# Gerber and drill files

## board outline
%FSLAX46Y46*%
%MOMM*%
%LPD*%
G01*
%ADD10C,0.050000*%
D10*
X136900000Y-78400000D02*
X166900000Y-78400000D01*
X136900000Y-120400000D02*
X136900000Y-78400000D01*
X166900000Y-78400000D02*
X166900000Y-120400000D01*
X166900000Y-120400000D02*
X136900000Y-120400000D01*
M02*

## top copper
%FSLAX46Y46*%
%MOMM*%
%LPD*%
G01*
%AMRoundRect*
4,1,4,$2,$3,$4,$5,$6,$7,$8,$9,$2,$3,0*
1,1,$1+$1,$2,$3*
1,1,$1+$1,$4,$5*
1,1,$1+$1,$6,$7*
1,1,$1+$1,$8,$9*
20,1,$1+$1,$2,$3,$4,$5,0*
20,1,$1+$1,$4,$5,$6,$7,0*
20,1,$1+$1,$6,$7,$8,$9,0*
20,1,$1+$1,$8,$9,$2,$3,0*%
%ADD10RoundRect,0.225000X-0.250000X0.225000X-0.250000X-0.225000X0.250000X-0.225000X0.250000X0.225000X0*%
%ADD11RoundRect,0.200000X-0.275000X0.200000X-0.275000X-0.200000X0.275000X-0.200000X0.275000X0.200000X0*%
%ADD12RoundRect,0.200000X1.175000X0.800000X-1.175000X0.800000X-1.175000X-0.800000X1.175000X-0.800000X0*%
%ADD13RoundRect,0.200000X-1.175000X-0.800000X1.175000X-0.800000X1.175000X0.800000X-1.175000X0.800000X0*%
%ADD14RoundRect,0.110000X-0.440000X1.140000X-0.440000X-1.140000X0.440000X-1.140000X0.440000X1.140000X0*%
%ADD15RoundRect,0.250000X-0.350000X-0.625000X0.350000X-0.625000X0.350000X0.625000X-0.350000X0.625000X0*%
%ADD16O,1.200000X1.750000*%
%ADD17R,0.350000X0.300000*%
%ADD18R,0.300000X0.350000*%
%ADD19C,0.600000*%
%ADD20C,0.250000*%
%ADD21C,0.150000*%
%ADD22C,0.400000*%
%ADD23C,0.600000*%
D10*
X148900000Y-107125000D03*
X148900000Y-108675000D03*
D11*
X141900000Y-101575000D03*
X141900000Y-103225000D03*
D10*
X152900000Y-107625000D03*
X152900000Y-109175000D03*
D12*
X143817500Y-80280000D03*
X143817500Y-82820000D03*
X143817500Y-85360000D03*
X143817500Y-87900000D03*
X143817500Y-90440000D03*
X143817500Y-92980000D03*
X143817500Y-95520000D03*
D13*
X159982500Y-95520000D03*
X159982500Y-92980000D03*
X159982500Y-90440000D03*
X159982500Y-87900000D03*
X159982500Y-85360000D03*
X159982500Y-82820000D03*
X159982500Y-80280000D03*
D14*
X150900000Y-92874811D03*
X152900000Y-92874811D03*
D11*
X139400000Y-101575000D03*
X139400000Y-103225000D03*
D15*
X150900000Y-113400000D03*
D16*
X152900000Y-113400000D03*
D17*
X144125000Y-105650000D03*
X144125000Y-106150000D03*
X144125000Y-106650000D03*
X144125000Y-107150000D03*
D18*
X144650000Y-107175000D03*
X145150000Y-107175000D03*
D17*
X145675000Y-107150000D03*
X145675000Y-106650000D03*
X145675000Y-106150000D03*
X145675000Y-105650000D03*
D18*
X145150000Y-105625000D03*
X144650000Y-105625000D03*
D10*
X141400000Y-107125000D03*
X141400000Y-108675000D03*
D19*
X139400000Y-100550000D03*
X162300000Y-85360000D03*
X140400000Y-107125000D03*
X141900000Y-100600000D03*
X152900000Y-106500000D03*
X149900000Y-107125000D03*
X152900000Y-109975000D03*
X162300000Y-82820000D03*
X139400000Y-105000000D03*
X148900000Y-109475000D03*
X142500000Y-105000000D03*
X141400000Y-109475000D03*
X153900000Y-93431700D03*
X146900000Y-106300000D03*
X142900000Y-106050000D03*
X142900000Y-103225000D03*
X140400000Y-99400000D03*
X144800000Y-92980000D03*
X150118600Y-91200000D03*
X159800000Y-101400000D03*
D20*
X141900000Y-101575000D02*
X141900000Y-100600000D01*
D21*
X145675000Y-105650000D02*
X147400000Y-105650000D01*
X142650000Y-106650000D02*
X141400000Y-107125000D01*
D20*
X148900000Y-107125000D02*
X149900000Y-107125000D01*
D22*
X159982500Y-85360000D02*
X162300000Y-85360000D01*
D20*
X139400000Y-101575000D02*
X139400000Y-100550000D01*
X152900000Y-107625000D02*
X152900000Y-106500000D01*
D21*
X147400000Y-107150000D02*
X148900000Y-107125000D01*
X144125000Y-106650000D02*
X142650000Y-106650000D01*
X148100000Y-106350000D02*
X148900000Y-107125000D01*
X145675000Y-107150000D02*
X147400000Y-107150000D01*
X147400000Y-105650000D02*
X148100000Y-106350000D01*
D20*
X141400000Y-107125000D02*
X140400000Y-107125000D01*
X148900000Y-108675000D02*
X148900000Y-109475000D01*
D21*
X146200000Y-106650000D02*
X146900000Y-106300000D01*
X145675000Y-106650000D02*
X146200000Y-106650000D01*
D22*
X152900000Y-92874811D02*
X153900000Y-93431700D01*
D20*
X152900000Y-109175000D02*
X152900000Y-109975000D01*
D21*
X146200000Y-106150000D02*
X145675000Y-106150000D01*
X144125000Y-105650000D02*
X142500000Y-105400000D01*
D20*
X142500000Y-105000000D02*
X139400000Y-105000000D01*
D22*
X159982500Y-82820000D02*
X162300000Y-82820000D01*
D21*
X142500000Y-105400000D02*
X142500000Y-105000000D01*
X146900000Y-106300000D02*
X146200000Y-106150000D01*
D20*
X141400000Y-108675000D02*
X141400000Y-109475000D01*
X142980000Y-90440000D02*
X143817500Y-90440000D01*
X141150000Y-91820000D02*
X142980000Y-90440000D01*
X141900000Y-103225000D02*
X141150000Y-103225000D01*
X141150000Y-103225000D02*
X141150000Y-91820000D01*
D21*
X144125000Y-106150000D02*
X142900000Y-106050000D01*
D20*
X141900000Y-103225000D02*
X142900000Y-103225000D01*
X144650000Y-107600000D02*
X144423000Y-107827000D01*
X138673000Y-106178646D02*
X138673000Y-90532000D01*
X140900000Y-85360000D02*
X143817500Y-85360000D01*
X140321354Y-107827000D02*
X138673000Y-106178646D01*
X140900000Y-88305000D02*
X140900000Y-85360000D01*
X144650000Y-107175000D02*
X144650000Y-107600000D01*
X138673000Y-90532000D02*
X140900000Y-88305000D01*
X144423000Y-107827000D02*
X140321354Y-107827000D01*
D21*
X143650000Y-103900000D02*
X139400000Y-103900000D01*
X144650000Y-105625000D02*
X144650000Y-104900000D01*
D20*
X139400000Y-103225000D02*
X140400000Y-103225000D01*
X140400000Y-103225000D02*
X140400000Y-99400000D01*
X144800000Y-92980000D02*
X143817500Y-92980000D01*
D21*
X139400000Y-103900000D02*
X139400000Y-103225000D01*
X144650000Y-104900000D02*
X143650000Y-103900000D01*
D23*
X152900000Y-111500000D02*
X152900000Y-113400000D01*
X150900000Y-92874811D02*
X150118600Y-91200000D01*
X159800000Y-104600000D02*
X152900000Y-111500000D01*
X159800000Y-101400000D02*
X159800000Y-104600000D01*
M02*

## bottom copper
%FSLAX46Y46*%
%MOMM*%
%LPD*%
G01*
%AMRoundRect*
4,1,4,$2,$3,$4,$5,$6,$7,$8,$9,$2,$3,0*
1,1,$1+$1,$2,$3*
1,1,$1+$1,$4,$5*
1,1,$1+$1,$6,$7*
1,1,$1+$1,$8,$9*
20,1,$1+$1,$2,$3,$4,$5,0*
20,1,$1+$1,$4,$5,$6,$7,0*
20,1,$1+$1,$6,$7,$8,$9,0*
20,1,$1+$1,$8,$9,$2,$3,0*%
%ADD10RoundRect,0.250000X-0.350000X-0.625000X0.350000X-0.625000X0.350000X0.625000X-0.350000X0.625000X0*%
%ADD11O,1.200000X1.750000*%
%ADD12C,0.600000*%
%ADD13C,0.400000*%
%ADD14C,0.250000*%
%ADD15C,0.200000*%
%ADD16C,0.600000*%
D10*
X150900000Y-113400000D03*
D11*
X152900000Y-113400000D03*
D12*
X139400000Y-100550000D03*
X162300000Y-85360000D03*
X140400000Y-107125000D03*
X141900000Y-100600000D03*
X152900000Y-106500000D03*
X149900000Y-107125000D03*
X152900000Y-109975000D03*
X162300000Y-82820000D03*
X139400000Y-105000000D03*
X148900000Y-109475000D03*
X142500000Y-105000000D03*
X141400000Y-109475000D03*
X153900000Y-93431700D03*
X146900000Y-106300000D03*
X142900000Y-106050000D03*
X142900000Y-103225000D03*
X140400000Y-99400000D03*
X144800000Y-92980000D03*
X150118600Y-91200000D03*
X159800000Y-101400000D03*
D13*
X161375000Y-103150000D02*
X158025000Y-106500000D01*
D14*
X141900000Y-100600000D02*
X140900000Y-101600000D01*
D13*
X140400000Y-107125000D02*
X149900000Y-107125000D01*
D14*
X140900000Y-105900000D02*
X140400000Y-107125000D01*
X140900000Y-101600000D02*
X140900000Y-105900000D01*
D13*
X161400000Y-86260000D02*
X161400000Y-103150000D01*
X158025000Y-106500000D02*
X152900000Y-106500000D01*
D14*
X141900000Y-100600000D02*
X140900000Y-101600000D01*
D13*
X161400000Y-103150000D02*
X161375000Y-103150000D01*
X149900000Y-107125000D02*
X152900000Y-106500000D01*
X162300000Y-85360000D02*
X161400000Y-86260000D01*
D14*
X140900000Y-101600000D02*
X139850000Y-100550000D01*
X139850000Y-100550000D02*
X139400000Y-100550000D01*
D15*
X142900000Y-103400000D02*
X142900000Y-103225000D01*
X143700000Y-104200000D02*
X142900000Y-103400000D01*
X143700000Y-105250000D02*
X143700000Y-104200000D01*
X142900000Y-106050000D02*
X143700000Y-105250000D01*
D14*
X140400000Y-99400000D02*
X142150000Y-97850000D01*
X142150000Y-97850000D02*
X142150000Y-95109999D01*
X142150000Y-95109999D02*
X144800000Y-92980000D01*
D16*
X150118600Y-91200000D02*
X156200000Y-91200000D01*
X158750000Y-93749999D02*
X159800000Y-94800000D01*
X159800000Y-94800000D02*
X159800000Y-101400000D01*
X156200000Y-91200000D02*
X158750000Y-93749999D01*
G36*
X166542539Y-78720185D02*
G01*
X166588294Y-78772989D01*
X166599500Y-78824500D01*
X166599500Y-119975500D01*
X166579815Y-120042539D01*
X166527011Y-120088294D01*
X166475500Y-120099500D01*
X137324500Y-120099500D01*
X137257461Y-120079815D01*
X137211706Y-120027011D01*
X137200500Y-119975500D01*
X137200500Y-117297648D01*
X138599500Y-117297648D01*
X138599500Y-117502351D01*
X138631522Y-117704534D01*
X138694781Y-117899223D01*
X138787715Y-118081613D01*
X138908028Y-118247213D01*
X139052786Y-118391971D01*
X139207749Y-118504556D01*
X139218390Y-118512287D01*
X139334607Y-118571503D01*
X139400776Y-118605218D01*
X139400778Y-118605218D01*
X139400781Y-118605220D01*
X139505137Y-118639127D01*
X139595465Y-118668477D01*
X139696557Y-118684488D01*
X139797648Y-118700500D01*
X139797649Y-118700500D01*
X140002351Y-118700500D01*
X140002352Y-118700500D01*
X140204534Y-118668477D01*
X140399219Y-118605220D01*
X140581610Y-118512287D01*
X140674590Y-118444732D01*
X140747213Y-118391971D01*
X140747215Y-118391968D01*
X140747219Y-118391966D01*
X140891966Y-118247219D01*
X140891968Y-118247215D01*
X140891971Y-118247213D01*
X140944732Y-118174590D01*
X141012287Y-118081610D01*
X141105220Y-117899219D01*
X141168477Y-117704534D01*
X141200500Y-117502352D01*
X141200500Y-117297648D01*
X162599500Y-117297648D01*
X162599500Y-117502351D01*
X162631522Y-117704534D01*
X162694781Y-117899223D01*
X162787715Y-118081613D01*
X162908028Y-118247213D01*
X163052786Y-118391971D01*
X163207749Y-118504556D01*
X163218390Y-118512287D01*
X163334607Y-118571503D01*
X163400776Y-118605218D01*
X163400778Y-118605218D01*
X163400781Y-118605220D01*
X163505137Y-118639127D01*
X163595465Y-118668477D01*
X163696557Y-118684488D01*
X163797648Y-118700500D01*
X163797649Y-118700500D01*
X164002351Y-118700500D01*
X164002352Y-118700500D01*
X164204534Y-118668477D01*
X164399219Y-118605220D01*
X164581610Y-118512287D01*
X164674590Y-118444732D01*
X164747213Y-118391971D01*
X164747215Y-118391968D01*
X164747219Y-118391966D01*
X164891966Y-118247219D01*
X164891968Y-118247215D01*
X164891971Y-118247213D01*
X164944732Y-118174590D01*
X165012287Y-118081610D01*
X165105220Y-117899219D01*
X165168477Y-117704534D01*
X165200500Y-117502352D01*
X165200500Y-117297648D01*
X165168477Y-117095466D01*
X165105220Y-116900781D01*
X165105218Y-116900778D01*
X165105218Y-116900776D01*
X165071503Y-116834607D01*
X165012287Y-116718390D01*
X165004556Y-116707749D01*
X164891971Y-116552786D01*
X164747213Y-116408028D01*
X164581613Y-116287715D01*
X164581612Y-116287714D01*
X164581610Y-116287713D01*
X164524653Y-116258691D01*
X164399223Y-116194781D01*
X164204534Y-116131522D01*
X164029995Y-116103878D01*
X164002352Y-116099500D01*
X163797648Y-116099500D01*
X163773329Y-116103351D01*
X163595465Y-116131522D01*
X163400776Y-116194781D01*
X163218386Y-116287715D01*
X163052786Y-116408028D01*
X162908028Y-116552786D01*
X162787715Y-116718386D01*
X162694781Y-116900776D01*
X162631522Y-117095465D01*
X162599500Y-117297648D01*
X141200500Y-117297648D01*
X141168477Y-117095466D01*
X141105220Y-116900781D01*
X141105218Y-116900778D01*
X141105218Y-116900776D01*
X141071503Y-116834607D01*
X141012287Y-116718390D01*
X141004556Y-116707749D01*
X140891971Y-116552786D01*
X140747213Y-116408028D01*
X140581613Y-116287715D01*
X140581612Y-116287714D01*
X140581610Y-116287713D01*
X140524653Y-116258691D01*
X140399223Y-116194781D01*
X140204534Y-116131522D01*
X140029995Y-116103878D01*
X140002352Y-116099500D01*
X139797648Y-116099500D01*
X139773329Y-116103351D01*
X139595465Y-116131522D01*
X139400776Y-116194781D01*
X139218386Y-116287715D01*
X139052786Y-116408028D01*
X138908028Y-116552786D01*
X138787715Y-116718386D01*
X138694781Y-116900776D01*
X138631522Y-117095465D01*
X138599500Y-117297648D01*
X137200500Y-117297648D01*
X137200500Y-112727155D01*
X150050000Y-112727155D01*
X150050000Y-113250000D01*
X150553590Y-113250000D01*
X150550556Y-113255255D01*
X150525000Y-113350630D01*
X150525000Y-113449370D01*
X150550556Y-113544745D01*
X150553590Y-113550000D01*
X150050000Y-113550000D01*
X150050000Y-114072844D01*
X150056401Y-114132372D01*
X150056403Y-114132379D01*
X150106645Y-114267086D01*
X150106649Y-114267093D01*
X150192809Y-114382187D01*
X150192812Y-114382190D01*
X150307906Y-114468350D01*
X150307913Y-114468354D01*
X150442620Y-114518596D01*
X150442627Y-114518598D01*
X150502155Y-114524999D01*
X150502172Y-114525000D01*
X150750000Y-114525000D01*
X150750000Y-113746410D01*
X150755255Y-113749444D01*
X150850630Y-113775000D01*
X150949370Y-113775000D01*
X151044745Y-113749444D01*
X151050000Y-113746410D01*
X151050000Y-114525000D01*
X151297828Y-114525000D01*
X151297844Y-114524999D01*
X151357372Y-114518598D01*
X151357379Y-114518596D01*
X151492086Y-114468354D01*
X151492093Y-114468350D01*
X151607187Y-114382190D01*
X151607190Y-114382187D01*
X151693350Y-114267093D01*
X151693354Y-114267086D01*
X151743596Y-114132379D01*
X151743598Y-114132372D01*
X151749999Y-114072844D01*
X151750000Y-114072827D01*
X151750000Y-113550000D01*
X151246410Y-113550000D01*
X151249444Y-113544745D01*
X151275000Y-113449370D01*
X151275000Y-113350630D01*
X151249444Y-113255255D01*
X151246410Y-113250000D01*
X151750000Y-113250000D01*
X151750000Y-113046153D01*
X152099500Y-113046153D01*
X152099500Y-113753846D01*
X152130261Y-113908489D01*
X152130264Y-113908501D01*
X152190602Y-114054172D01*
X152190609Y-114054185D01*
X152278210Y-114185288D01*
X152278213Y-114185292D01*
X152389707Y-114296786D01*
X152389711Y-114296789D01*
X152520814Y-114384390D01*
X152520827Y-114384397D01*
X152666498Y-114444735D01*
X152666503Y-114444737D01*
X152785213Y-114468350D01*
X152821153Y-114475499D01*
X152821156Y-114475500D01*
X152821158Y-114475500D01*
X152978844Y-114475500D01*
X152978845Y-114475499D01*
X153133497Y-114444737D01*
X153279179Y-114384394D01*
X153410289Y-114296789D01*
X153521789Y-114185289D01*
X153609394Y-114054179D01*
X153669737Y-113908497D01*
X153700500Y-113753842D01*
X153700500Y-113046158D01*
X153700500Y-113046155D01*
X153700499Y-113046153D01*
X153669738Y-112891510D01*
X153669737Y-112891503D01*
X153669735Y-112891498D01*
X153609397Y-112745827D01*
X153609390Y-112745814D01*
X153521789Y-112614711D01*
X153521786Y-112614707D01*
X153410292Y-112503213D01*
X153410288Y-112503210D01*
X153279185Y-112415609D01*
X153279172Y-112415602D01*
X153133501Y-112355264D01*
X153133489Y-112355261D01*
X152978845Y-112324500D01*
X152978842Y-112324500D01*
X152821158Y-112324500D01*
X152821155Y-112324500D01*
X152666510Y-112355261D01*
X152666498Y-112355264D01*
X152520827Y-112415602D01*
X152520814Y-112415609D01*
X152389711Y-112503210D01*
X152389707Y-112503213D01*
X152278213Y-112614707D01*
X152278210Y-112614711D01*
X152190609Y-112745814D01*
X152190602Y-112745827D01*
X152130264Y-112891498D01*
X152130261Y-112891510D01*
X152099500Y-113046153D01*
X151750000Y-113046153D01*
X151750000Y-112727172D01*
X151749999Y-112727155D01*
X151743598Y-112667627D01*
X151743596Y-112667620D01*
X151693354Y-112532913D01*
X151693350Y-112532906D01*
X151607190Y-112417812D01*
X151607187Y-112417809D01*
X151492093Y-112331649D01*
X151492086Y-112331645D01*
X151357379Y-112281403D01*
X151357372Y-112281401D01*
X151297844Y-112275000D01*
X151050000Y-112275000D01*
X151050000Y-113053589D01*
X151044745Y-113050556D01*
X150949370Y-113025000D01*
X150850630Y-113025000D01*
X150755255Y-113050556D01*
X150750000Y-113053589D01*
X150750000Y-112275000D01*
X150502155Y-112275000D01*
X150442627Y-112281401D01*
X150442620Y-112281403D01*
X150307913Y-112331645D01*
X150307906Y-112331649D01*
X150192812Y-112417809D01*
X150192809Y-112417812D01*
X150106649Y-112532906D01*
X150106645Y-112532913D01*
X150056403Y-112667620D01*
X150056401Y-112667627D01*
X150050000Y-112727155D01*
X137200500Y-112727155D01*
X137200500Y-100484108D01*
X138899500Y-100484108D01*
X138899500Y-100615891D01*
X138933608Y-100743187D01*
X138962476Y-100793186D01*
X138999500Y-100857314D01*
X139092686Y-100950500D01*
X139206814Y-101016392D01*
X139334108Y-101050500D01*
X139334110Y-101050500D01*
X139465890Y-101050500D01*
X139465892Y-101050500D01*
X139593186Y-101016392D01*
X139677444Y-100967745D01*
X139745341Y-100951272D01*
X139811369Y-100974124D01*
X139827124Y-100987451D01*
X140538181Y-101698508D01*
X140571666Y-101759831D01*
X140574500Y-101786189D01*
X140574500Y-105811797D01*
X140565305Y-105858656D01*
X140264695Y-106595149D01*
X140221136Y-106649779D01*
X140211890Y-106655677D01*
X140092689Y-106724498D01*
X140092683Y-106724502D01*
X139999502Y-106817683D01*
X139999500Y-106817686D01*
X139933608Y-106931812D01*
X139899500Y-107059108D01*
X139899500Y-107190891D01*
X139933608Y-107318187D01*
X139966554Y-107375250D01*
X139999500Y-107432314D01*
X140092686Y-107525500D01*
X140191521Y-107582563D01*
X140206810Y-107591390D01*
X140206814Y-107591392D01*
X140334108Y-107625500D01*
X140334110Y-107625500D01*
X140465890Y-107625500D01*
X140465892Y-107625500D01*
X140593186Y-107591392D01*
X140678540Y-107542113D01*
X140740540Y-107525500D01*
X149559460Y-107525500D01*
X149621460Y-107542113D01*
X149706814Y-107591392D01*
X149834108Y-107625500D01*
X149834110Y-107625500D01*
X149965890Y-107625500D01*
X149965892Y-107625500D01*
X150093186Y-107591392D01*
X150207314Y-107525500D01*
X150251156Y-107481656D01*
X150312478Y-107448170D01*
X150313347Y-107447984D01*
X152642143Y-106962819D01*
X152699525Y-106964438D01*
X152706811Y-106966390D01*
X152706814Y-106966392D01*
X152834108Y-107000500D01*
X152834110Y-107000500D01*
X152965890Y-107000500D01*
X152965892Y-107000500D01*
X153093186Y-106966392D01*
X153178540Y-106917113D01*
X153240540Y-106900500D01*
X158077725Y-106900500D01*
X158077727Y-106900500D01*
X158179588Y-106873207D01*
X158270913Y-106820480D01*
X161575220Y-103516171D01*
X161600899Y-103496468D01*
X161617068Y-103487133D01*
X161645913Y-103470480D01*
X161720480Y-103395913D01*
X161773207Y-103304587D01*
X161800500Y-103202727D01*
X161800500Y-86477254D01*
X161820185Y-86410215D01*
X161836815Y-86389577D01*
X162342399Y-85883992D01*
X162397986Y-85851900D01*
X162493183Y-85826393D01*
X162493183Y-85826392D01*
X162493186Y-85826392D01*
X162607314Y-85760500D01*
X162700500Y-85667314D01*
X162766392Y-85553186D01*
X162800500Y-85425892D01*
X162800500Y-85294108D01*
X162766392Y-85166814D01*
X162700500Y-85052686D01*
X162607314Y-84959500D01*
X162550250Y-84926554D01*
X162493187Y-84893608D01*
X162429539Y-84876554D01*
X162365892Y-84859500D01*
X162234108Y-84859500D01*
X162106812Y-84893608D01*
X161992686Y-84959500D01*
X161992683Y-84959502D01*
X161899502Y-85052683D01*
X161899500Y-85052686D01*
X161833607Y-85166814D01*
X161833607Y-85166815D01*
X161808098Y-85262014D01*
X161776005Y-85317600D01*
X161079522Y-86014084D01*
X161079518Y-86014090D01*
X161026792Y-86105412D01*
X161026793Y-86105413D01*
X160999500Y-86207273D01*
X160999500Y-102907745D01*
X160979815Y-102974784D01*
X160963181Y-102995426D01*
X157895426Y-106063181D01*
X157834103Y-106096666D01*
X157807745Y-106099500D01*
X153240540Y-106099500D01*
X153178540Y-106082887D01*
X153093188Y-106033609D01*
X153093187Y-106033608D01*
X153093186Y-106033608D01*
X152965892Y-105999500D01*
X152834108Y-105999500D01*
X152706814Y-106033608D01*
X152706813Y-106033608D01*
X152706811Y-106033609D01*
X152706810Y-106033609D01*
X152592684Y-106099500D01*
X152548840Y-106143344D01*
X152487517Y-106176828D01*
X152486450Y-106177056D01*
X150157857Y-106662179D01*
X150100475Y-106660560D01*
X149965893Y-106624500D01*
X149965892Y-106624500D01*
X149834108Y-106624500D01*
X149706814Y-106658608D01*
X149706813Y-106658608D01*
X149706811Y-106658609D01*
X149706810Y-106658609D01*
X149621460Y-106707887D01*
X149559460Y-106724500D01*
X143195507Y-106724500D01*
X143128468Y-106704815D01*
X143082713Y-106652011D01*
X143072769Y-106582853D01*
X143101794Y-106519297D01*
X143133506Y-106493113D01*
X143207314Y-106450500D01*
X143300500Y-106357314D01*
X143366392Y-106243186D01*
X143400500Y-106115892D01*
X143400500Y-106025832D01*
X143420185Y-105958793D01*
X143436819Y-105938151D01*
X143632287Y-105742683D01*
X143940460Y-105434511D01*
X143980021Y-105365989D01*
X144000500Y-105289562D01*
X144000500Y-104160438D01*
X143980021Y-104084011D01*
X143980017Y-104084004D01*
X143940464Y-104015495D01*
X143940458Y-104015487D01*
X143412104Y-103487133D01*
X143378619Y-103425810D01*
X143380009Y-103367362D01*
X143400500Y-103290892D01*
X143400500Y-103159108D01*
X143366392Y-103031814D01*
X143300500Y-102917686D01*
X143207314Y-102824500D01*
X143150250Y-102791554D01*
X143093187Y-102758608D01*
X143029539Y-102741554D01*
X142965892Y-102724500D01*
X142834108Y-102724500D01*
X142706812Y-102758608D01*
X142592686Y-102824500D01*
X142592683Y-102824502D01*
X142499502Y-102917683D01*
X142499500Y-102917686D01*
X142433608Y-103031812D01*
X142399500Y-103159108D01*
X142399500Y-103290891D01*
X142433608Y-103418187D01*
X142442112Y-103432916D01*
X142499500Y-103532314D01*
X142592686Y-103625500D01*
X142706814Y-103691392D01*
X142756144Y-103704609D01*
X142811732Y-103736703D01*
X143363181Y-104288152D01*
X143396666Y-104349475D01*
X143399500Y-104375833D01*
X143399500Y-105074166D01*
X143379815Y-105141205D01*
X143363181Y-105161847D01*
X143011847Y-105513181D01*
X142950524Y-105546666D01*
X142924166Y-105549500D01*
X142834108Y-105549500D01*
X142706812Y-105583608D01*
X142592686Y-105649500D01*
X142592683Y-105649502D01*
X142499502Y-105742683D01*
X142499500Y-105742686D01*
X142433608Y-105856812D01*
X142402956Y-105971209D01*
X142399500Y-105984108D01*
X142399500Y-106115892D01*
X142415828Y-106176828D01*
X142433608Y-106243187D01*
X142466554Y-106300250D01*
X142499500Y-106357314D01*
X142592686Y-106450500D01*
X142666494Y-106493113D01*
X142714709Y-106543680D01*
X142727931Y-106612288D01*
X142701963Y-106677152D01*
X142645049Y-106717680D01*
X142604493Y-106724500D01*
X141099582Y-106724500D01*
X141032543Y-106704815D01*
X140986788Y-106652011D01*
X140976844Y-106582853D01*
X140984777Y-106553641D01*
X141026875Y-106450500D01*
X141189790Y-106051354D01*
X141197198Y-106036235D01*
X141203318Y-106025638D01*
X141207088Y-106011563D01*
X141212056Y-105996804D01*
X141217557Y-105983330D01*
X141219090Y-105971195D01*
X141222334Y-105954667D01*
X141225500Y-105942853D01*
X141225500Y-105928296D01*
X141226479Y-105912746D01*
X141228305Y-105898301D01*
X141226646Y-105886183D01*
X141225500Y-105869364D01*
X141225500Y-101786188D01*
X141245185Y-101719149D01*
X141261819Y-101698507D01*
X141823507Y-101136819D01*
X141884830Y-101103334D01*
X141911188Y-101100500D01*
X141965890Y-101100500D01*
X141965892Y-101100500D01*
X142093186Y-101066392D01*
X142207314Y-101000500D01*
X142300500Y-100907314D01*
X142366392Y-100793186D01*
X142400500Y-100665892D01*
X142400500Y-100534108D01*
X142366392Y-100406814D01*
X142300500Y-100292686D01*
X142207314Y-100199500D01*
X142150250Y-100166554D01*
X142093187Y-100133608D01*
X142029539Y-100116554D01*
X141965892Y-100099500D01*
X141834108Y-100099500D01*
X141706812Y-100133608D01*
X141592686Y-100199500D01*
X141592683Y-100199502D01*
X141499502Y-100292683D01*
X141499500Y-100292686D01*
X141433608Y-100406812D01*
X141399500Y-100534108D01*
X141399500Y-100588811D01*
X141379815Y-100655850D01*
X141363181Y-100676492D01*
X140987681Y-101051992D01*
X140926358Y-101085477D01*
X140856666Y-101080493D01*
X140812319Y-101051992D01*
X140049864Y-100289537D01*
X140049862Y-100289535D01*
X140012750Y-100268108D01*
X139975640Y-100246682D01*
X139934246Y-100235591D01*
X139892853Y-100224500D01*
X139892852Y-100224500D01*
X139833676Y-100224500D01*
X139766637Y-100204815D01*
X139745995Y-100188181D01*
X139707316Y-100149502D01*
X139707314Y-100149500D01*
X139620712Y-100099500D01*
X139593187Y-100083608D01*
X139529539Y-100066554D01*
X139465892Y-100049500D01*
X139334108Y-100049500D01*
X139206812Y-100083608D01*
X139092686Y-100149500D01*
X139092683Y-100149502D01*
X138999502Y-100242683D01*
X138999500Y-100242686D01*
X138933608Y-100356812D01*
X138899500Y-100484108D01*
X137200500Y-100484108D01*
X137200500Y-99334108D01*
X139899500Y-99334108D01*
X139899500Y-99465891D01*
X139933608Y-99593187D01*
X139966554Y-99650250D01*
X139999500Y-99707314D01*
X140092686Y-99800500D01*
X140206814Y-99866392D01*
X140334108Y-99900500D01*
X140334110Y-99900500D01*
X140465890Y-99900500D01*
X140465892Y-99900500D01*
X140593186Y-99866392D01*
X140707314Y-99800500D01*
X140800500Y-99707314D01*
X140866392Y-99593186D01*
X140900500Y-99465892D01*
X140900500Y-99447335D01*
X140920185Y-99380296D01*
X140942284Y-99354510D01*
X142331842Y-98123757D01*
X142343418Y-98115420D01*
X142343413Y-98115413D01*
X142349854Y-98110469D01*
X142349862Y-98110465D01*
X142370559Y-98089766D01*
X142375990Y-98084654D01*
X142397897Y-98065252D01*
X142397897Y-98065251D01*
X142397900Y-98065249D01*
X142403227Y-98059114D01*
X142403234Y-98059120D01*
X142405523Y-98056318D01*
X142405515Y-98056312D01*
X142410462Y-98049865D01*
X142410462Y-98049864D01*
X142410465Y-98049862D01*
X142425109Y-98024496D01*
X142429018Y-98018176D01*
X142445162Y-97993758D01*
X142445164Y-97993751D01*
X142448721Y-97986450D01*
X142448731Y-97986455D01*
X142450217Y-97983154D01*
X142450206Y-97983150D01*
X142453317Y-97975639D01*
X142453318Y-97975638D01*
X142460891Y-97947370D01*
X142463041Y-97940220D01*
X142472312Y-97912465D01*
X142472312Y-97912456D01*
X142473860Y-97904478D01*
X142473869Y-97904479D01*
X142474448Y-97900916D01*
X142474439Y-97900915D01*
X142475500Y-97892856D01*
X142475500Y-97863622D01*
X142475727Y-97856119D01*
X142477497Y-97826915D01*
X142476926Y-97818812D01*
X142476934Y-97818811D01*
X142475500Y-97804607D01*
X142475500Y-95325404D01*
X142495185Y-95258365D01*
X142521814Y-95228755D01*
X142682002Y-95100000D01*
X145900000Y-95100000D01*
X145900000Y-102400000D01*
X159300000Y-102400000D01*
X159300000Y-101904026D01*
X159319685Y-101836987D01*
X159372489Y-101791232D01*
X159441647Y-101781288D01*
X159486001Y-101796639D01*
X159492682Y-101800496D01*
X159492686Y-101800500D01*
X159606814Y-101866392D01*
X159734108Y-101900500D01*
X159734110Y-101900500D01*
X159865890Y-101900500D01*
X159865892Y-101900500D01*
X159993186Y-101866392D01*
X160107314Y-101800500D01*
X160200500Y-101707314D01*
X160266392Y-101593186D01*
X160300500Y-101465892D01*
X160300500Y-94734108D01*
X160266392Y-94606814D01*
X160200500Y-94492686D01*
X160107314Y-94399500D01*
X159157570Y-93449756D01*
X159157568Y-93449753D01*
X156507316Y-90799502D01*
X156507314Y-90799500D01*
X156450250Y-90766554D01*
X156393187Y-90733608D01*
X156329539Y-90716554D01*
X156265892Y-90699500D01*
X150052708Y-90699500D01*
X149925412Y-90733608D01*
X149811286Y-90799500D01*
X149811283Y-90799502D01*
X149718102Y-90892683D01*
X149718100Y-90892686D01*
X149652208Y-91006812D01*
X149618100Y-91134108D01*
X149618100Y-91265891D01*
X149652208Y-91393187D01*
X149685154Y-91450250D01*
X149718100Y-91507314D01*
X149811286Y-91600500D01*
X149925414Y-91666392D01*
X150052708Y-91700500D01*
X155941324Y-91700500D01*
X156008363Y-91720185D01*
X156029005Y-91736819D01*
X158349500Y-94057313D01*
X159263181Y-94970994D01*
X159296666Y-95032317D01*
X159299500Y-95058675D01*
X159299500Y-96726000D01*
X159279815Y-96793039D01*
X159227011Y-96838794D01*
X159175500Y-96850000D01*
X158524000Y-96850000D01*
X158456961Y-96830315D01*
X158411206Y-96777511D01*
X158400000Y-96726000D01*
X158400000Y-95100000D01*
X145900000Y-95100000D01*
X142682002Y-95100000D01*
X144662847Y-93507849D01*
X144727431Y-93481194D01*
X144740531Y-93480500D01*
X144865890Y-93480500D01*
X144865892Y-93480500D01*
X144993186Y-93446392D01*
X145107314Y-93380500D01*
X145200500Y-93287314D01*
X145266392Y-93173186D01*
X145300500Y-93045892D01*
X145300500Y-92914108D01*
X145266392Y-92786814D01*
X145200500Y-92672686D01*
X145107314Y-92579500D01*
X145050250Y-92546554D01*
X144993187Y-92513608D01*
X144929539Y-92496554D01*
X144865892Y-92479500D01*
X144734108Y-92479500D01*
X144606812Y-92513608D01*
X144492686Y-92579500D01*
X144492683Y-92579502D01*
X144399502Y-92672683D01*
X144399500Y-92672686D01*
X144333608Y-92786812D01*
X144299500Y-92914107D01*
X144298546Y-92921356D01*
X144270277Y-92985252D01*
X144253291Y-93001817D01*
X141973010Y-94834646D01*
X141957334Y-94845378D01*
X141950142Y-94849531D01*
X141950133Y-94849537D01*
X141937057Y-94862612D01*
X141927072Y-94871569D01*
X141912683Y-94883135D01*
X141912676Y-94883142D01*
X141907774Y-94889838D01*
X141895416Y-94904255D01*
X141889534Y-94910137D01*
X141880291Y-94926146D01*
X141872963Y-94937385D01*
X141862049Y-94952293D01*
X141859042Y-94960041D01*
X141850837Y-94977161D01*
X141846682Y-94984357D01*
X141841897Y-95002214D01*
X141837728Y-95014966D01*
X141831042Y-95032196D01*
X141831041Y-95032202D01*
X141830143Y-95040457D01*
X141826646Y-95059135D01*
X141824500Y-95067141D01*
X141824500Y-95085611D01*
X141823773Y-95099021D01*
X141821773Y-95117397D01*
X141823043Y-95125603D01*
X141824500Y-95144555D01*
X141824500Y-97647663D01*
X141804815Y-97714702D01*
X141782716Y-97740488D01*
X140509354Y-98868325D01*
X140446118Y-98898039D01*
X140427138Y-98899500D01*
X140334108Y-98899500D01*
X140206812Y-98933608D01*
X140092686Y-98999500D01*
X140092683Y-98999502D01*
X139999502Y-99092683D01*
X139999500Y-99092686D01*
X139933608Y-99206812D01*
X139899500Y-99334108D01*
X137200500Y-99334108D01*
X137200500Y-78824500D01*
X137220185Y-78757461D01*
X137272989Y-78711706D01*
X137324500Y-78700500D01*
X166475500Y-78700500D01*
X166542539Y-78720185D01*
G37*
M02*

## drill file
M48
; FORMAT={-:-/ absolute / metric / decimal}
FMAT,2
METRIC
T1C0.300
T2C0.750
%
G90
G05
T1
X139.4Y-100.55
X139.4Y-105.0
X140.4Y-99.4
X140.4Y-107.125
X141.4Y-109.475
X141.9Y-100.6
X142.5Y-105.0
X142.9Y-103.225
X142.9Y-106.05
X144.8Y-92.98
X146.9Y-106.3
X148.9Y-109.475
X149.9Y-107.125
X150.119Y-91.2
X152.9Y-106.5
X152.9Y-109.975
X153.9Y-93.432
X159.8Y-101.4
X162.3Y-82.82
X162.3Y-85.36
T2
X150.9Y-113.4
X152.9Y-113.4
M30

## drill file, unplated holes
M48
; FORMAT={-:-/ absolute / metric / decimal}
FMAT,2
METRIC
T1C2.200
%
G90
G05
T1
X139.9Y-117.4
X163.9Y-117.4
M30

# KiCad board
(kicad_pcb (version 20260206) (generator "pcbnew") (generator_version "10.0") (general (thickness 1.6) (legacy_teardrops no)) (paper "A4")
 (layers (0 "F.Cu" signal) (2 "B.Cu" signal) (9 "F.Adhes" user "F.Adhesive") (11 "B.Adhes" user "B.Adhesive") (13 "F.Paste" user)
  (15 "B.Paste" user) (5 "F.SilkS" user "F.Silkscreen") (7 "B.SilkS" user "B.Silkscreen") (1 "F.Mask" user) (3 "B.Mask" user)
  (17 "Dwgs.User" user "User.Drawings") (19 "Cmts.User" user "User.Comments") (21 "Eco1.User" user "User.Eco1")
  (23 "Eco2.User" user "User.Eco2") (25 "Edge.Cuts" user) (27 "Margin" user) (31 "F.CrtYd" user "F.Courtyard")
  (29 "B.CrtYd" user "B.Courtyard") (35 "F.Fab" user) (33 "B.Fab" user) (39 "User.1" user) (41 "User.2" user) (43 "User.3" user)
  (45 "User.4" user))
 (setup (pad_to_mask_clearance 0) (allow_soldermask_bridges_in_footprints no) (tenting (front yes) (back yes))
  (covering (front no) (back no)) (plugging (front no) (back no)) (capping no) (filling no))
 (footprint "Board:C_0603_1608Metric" (layer "F.Cu") (at 148.9 107.9 -90)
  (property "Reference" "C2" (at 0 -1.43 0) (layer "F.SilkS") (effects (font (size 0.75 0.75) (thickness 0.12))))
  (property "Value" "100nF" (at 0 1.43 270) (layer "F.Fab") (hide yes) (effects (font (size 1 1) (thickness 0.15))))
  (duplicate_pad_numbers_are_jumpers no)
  (pad "1" smd roundrect (at -0.775 0 270) (size 0.9 0.95) (layers "F.Cu" "F.Mask" "F.Paste") (roundrect_rratio 0.25) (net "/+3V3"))
  (pad "2" smd roundrect (at 0.775 0 270) (size 0.9 0.95) (layers "F.Cu" "F.Mask" "F.Paste") (roundrect_rratio 0.25) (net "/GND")))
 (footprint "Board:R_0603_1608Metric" (layer "F.Cu") (at 141.9 102.4 -90)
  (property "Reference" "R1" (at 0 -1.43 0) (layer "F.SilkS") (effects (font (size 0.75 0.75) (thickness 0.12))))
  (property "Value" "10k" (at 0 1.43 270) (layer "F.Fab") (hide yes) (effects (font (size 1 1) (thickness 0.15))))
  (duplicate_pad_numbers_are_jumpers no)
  (pad "1" smd roundrect (at -0.825 0 270) (size 0.8 0.95) (layers "F.Cu" "F.Mask" "F.Paste") (roundrect_rratio 0.25) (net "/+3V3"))
  (pad "2" smd roundrect (at 0.825 0 270) (size 0.8 0.95) (layers "F.Cu" "F.Mask" "F.Paste") (roundrect_rratio 0.25) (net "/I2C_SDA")))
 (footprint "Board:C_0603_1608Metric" (layer "F.Cu") (at 152.9 108.4 -90)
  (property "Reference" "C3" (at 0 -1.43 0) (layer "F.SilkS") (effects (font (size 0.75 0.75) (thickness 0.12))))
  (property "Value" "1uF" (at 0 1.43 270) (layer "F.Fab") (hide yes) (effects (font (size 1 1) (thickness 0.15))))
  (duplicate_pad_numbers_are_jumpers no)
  (pad "1" smd roundrect (at -0.775 0 270) (size 0.9 0.95) (layers "F.Cu" "F.Mask" "F.Paste") (roundrect_rratio 0.25) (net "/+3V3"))
  (pad "2" smd roundrect (at 0.775 0 270) (size 0.9 0.95) (layers "F.Cu" "F.Mask" "F.Paste") (roundrect_rratio 0.25) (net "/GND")))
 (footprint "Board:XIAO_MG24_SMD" (layer "F.Cu") (at 151.9 87.9 90)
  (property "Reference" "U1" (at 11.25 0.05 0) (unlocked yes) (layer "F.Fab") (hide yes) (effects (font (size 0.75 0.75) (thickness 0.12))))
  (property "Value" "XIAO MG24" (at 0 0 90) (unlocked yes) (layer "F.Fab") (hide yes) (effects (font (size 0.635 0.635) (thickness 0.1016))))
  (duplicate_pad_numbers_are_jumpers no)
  (pad "1" smd roundrect (at 7.62 -8.0825 180) (size 2.75 2) (layers "F.Cu" "F.Mask" "F.Paste") (roundrect_rratio 0.1)
   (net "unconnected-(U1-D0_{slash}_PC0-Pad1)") (thermal_bridge_angle 45))
  (pad "2" smd roundrect (at 5.08 -8.0825 180) (size 2.75 2) (layers "F.Cu" "F.Mask" "F.Paste") (roundrect_rratio 0.1)
   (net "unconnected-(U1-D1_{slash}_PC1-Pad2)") (thermal_bridge_angle 45))
  (pad "3" smd roundrect (at 2.54 -8.0825 180) (size 2.75 2) (layers "F.Cu" "F.Mask" "F.Paste") (roundrect_rratio 0.1) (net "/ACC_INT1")
   (thermal_bridge_angle 45))
  (pad "4" smd roundrect (at 0 -8.0825 180) (size 2.75 2) (layers "F.Cu" "F.Mask" "F.Paste") (roundrect_rratio 0.1)
   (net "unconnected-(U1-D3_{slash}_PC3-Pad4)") (thermal_bridge_angle 45))
  (pad "5" smd roundrect (at -2.54 -8.0825 180) (size 2.75 2) (layers "F.Cu" "F.Mask" "F.Paste") (roundrect_rratio 0.1) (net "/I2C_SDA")
   (thermal_bridge_angle 45))
  (pad "6" smd roundrect (at -5.08 -8.0825 180) (size 2.75 2) (layers "F.Cu" "F.Mask" "F.Paste") (roundrect_rratio 0.1) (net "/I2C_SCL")
   (thermal_bridge_angle 45))
  (pad "7" smd roundrect (at -7.62 -8.0825 180) (size 2.75 2) (layers "F.Cu" "F.Mask" "F.Paste") (roundrect_rratio 0.1)
   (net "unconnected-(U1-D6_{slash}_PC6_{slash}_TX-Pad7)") (thermal_bridge_angle 45))
  (pad "8" smd roundrect (at -7.62 8.0825) (size 2.75 2) (layers "F.Cu" "F.Mask" "F.Paste") (roundrect_rratio 0.1)
   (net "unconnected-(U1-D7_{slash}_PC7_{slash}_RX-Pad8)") (thermal_bridge_angle 45))
  (pad "9" smd roundrect (at -5.08 8.0825) (size 2.75 2) (layers "F.Cu" "F.Mask" "F.Paste") (roundrect_rratio 0.1)
   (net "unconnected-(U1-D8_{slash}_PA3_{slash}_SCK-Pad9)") (thermal_bridge_angle 45))
  (pad "10" smd roundrect (at -2.54 8.0825) (size 2.75 2) (layers "F.Cu" "F.Mask" "F.Paste") (roundrect_rratio 0.1)
   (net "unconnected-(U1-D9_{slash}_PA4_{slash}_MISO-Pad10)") (thermal_bridge_angle 45))
  (pad "11" smd roundrect (at 0 8.0825) (size 2.75 2) (layers "F.Cu" "F.Mask" "F.Paste") (roundrect_rratio 0.1)
   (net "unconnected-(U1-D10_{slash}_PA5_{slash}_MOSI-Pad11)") (thermal_bridge_angle 45))
  (pad "12" smd roundrect (at 2.54 8.0825) (size 2.75 2) (layers "F.Cu" "F.Mask" "F.Paste") (roundrect_rratio 0.1) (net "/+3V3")
   (thermal_bridge_angle 45))
  (pad "13" smd roundrect (at 5.08 8.0825) (size 2.75 2) (layers "F.Cu" "F.Mask" "F.Paste") (roundrect_rratio 0.1) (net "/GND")
   (thermal_bridge_angle 45))
  (pad "14" smd roundrect (at 7.62 8.0825) (size 2.75 2) (layers "F.Cu" "F.Mask" "F.Paste") (roundrect_rratio 0.1)
   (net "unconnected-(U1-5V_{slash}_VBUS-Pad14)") (thermal_bridge_angle 45))
  (pad "31" smd roundrect (at -4.974811 -1 270) (size 2.5 1.1) (layers "F.Cu" "F.Mask" "F.Paste") (roundrect_rratio 0.1) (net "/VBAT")
   (thermal_bridge_angle 45))
  (pad "32" smd roundrect (at -4.974811 1 270) (size 2.5 1.1) (layers "F.Cu" "F.Mask" "F.Paste") (roundrect_rratio 0.1) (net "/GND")
   (thermal_bridge_angle 45)))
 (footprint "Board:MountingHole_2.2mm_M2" (layer "F.Cu") (at 139.9 117.4)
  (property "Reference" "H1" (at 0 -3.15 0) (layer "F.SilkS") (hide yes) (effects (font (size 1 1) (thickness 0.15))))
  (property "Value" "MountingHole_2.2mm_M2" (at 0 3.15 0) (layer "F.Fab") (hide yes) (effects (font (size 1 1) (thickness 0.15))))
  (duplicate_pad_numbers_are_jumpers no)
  (pad "" np_thru_hole circle (at 0 0) (size 2.2 2.2) (drill 2.2) (layers "*.Cu" "*.Mask")))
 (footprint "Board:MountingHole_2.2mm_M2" (layer "F.Cu") (at 163.9 117.4)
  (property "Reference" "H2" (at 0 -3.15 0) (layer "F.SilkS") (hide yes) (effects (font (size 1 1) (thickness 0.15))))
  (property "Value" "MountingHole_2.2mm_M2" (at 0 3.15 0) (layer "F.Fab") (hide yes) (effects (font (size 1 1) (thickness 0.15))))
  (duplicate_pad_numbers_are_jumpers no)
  (pad "" np_thru_hole circle (at 0 0) (size 2.2 2.2) (drill 2.2) (layers "*.Cu" "*.Mask")))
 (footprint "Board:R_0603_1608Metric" (layer "F.Cu") (at 139.4 102.4 -90)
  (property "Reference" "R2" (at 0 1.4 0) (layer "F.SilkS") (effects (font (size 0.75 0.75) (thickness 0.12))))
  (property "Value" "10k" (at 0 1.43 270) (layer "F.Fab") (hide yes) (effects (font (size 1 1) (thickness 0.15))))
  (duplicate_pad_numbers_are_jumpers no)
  (pad "1" smd roundrect (at -0.825 0 270) (size 0.8 0.95) (layers "F.Cu" "F.Mask" "F.Paste") (roundrect_rratio 0.25) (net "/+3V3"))
  (pad "2" smd roundrect (at 0.825 0 270) (size 0.8 0.95) (layers "F.Cu" "F.Mask" "F.Paste") (roundrect_rratio 0.25) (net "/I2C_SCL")))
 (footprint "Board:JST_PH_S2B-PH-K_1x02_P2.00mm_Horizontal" (layer "F.Cu") (at 150.9 113.4)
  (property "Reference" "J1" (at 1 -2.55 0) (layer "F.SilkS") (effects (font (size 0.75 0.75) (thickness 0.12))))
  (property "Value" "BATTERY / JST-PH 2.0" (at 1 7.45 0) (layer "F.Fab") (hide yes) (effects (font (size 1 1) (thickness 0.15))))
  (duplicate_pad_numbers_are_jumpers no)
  (pad "1" thru_hole roundrect (at 0 0) (size 1.2 1.75) (drill 0.75) (layers "*.Cu" "*.Mask") (remove_unused_layers no)
   (roundrect_rratio 0.208333) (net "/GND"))
  (pad "2" thru_hole oval (at 2 0) (size 1.2 1.75) (drill 0.75) (layers "*.Cu" "*.Mask") (remove_unused_layers no) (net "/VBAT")))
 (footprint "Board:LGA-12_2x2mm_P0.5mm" (layer "F.Cu") (at 144.9 106.4)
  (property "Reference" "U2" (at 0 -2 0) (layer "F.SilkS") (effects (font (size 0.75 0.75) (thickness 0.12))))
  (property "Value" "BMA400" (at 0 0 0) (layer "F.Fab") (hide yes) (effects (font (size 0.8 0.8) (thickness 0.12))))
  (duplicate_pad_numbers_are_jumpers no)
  (pad "1" smd rect (at -0.775 -0.75) (size 0.35 0.3) (layers "F.Cu" "F.Mask" "F.Paste") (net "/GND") (solder_mask_margin 0.05)
   (solder_paste_margin -0.025))
  (pad "2" smd rect (at -0.775 -0.25) (size 0.35 0.3) (layers "F.Cu" "F.Mask" "F.Paste") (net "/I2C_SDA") (solder_mask_margin 0.05)
   (solder_paste_margin -0.025))
  (pad "3" smd rect (at -0.775 0.25) (size 0.35 0.3) (layers "F.Cu" "F.Mask" "F.Paste") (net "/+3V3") (solder_mask_margin 0.05)
   (solder_paste_margin -0.025))
  (pad "4" smd rect (at -0.775 0.75) (size 0.35 0.3) (layers "F.Cu" "F.Mask" "F.Paste") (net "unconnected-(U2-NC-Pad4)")
   (solder_mask_margin 0.05) (solder_paste_margin -0.025))
  (pad "5" smd rect (at -0.25 0.775) (size 0.3 0.35) (layers "F.Cu" "F.Mask" "F.Paste") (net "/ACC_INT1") (solder_mask_margin 0.05)
   (solder_paste_margin -0.025))
  (pad "6" smd rect (at 0.25 0.775) (size 0.3 0.35) (layers "F.Cu" "F.Mask" "F.Paste") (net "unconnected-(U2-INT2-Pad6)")
   (solder_mask_margin 0.05) (solder_paste_margin -0.025))
  (pad "7" smd rect (at 0.775 0.75) (size 0.35 0.3) (layers "F.Cu" "F.Mask" "F.Paste") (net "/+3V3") (solder_mask_margin 0.05)
   (solder_paste_margin -0.025))
  (pad "8" smd rect (at 0.775 0.25) (size 0.35 0.3) (layers "F.Cu" "F.Mask" "F.Paste") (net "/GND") (solder_mask_margin 0.05)
   (solder_paste_margin -0.025))
  (pad "9" smd rect (at 0.775 -0.25) (size 0.35 0.3) (layers "F.Cu" "F.Mask" "F.Paste") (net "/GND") (solder_mask_margin 0.05)
   (solder_paste_margin -0.025))
  (pad "10" smd rect (at 0.775 -0.75) (size 0.35 0.3) (layers "F.Cu" "F.Mask" "F.Paste") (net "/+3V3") (solder_mask_margin 0.05)
   (solder_paste_margin -0.025))
  (pad "11" smd rect (at 0.25 -0.775) (size 0.3 0.35) (layers "F.Cu" "F.Mask" "F.Paste") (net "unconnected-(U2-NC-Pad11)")
   (solder_mask_margin 0.05) (solder_paste_margin -0.025))
  (pad "12" smd rect (at -0.25 -0.775) (size 0.3 0.35) (layers "F.Cu" "F.Mask" "F.Paste") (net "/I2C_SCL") (solder_mask_margin 0.05)
   (solder_paste_margin -0.025)))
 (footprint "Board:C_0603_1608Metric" (layer "F.Cu") (at 141.4 107.9 -90)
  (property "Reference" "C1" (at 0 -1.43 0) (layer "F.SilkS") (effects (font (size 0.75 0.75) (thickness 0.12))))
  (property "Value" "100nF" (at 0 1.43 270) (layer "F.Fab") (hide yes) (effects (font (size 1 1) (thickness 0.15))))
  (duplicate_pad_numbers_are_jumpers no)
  (pad "1" smd roundrect (at -0.775 0 270) (size 0.9 0.95) (layers "F.Cu" "F.Mask" "F.Paste") (roundrect_rratio 0.25) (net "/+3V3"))
  (pad "2" smd roundrect (at 0.775 0 270) (size 0.9 0.95) (layers "F.Cu" "F.Mask" "F.Paste") (roundrect_rratio 0.25) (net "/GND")))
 (gr_line (start 136.9 78.4) (end 166.9 78.4) (stroke (width 0.05) (type default)) (layer "Edge.Cuts"))
 (gr_line (start 136.9 120.4) (end 136.9 78.4) (stroke (width 0.05) (type default)) (layer "Edge.Cuts"))
 (gr_line (start 166.9 78.4) (end 166.9 120.4) (stroke (width 0.05) (type default)) (layer "Edge.Cuts"))
 (gr_line (start 166.9 120.4) (end 136.9 120.4) (stroke (width 0.05) (type default)) (layer "Edge.Cuts"))
 (segment (start 141.9 101.575) (end 141.9 100.6) (width 0.25) (layer "F.Cu") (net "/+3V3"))
 (segment (start 145.675 105.65) (end 147.4 105.65) (width 0.15) (layer "F.Cu") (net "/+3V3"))
 (segment (start 142.65 106.65) (end 141.4 107.125) (width 0.15) (layer "F.Cu") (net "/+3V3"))
 (segment (start 148.9 107.125) (end 149.9 107.125) (width 0.25) (layer "F.Cu") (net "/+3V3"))
 (segment (start 159.9825 85.36) (end 162.3 85.36) (width 0.4) (layer "F.Cu") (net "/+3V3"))
 (segment (start 139.4 101.575) (end 139.4 100.55) (width 0.25) (layer "F.Cu") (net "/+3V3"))
 (segment (start 152.9 107.625) (end 152.9 106.5) (width 0.25) (layer "F.Cu") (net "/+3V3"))
 (segment (start 147.4 107.15) (end 148.9 107.125) (width 0.15) (layer "F.Cu") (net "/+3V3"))
 (segment (start 144.125 106.65) (end 142.65 106.65) (width 0.15) (layer "F.Cu") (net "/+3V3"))
 (segment (start 148.1 106.35) (end 148.9 107.125) (width 0.15) (layer "F.Cu") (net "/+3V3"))
 (segment (start 145.675 107.15) (end 147.4 107.15) (width 0.15) (layer "F.Cu") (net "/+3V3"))
 (segment (start 147.4 105.65) (end 148.1 106.35) (width 0.15) (layer "F.Cu") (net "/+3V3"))
 (segment (start 141.4 107.125) (end 140.4 107.125) (width 0.25) (layer "F.Cu") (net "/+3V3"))
 (via (at 139.4 100.55) (size 0.6) (drill 0.3) (layers "F.Cu" "B.Cu") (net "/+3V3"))
 (via (at 162.3 85.36) (size 0.6) (drill 0.3) (layers "F.Cu" "B.Cu") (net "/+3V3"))
 (via (at 140.4 107.125) (size 0.6) (drill 0.3) (layers "F.Cu" "B.Cu") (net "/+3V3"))
 (via (at 141.9 100.6) (size 0.6) (drill 0.3) (layers "F.Cu" "B.Cu") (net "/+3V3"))
 (via (at 152.9 106.5) (size 0.6) (drill 0.3) (layers "F.Cu" "B.Cu") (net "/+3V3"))
 (via (at 149.9 107.125) (size 0.6) (drill 0.3) (layers "F.Cu" "B.Cu") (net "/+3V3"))
 (segment (start 161.375 103.15) (end 158.025 106.5) (width 0.4) (layer "B.Cu") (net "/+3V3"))
 (segment (start 141.9 100.6) (end 140.9 101.6) (width 0.25) (layer "B.Cu") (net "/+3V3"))
 (segment (start 140.4 107.125) (end 149.9 107.125) (width 0.4) (layer "B.Cu") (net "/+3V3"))
 (segment (start 140.9 105.9) (end 140.4 107.125) (width 0.25) (layer "B.Cu") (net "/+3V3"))
 (segment (start 140.9 101.6) (end 140.9 105.9) (width 0.25) (layer "B.Cu") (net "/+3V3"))
 (segment (start 161.4 86.26) (end 161.4 103.15) (width 0.4) (layer "B.Cu") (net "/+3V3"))
 (segment (start 158.025 106.5) (end 152.9 106.5) (width 0.4) (layer "B.Cu") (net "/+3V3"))
 (segment (start 141.9 100.6) (end 140.9 101.6) (width 0.25) (layer "B.Cu") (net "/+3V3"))
 (segment (start 161.4 103.15) (end 161.375 103.15) (width 0.4) (layer "B.Cu") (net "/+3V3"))
 (segment (start 149.9 107.125) (end 152.9 106.5) (width 0.4) (layer "B.Cu") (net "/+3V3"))
 (segment (start 162.3 85.36) (end 161.4 86.26) (width 0.4) (layer "B.Cu") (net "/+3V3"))
 (segment (start 140.9 101.6) (end 139.85 100.55) (width 0.25) (layer "B.Cu") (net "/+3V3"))
 (segment (start 139.85 100.55) (end 139.4 100.55) (width 0.25) (layer "B.Cu") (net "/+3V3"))
 (segment (start 148.9 108.675) (end 148.9 109.475) (width 0.25) (layer "F.Cu") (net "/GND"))
 (segment (start 146.2 106.65) (end 146.9 106.3) (width 0.15) (layer "F.Cu") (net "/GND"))
 (segment (start 145.675 106.65) (end 146.2 106.65) (width 0.15) (layer "F.Cu") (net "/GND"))
 (segment (start 152.9 92.874811) (end 153.9 93.4317) (width 0.4) (layer "F.Cu") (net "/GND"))
 (segment (start 152.9 109.175) (end 152.9 109.975) (width 0.25) (layer "F.Cu") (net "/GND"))
 (segment (start 146.2 106.15) (end 145.675 106.15) (width 0.15) (layer "F.Cu") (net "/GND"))
 (segment (start 144.125 105.65) (end 142.5 105.4) (width 0.15) (layer "F.Cu") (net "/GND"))
 (segment (start 142.5 105) (end 139.4 105) (width 0.25) (layer "F.Cu") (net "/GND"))
 (segment (start 159.9825 82.82) (end 162.3 82.82) (width 0.4) (layer "F.Cu") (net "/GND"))
 (segment (start 142.5 105.4) (end 142.5 105) (width 0.15) (layer "F.Cu") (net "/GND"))
 (segment (start 146.9 106.3) (end 146.2 106.15) (width 0.15) (layer "F.Cu") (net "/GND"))
 (segment (start 141.4 108.675) (end 141.4 109.475) (width 0.25) (layer "F.Cu") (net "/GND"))
 (via (at 152.9 109.975) (size 0.6) (drill 0.3) (layers "F.Cu" "B.Cu") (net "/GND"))
 (via (at 162.3 82.82) (size 0.6) (drill 0.3) (layers "F.Cu" "B.Cu") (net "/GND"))
 (via (at 139.4 105) (size 0.6) (drill 0.3) (layers "F.Cu" "B.Cu") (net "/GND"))
 (via (at 148.9 109.475) (size 0.6) (drill 0.3) (layers "F.Cu" "B.Cu") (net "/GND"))
 (via (at 142.5 105) (size 0.6) (drill 0.3) (layers "F.Cu" "B.Cu") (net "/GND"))
 (via (at 141.4 109.475) (size 0.6) (drill 0.3) (layers "F.Cu" "B.Cu") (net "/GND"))
 (via (at 153.9 93.4317) (size 0.6) (drill 0.3) (layers "F.Cu" "B.Cu") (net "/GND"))
 (via (at 146.9 106.3) (size 0.6) (drill 0.3) (layers "F.Cu" "B.Cu") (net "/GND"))
 (segment (start 142.98 90.44) (end 143.8175 90.44) (width 0.25) (layer "F.Cu") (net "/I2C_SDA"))
 (segment (start 141.15 91.82) (end 142.98 90.44) (width 0.25) (layer "F.Cu") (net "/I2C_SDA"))
 (segment (start 141.9 103.225) (end 141.15 103.225) (width 0.25) (layer "F.Cu") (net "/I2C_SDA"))
 (segment (start 141.15 103.225) (end 141.15 91.82) (width 0.25) (layer "F.Cu") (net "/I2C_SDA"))
 (segment (start 144.125 106.15) (end 142.9 106.05) (width 0.15) (layer "F.Cu") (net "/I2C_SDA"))
 (segment (start 141.9 103.225) (end 142.9 103.225) (width 0.25) (layer "F.Cu") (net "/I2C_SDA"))
 (via (at 142.9 106.05) (size 0.6) (drill 0.3) (layers "F.Cu" "B.Cu") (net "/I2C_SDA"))
 (via (at 142.9 103.225) (size 0.6) (drill 0.3) (layers "F.Cu" "B.Cu") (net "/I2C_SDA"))
 (segment (start 142.9 103.4) (end 142.9 103.225) (width 0.2) (layer "B.Cu") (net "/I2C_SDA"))
 (segment (start 143.7 104.2) (end 142.9 103.4) (width 0.2) (layer "B.Cu") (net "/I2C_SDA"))
 (segment (start 143.7 105.25) (end 143.7 104.2) (width 0.2) (layer "B.Cu") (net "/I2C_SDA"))
 (segment (start 142.9 106.05) (end 143.7 105.25) (width 0.2) (layer "B.Cu") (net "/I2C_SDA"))
 (segment (start 144.65 107.6) (end 144.423 107.827) (width 0.25) (layer "F.Cu") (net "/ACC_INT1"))
 (segment (start 138.673 106.178646) (end 138.673 90.532) (width 0.25) (layer "F.Cu") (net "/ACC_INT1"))
 (segment (start 140.321354 107.827) (end 138.673 106.178646) (width 0.25) (layer "F.Cu") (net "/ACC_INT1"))
 (segment (start 143.8175 85.36) (end 142.4425 85.36) (width 0.25) (layer "F.Cu") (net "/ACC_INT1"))
 (segment (start 144.65 107.175) (end 144.65 107.6) (width 0.25) (layer "F.Cu") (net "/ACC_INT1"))
 (segment (start 144.423 107.827) (end 140.321354 107.827) (width 0.25) (layer "F.Cu") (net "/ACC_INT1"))
 (segment (start 142.4425 85.36) (end 138.673 89.1295) (width 0.25) (layer "F.Cu") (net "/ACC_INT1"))
 (segment (start 138.673 89.1295) (end 138.673 90.532) (width 0.25) (layer "F.Cu") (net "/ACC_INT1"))
 (segment (start 143.65 103.9) (end 139.4 103.9) (width 0.15) (layer "F.Cu") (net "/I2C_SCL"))
 (segment (start 144.65 105.625) (end 144.65 104.9) (width 0.15) (layer "F.Cu") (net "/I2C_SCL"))
 (segment (start 139.4 103.225) (end 140.4 103.225) (width 0.25) (layer "F.Cu") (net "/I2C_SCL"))
 (segment (start 140.4 103.225) (end 140.4 99.4) (width 0.25) (layer "F.Cu") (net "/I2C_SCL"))
 (segment (start 144.8 92.98) (end 143.8175 92.98) (width 0.25) (layer "F.Cu") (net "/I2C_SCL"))
 (segment (start 139.4 103.9) (end 139.4 103.225) (width 0.15) (layer "F.Cu") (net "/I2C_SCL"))
 (segment (start 144.65 104.9) (end 143.65 103.9) (width 0.15) (layer "F.Cu") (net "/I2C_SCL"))
 (via (at 140.4 99.4) (size 0.6) (drill 0.3) (layers "F.Cu" "B.Cu") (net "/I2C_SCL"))
 (via (at 144.8 92.98) (size 0.6) (drill 0.3) (layers "F.Cu" "B.Cu") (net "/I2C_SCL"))
 (segment (start 140.4 99.4) (end 142.15 97.85) (width 0.25) (layer "B.Cu") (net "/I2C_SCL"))
 (segment (start 142.15 97.85) (end 142.15 95.109999) (width 0.25) (layer "B.Cu") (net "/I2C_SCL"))
 (segment (start 142.15 95.109999) (end 144.8 92.98) (width 0.25) (layer "B.Cu") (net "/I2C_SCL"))
 (segment (start 152.9 111.5) (end 152.9 113.4) (width 0.6) (layer "F.Cu") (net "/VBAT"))
 (segment (start 150.9 92.874811) (end 150.1186 91.2) (width 0.6) (layer "F.Cu") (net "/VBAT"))
 (segment (start 159.8 104.6) (end 152.9 111.5) (width 0.6) (layer "F.Cu") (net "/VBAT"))
 (segment (start 159.8 101.4) (end 159.8 104.6) (width 0.6) (layer "F.Cu") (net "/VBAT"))
 (via (at 150.1186 91.2) (size 0.6) (drill 0.3) (layers "F.Cu" "B.Cu") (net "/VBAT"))
 (via (at 159.8 101.4) (size 0.6) (drill 0.3) (layers "F.Cu" "B.Cu") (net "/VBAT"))
 (segment (start 150.1186 91.2) (end 156.2 91.2) (width 0.6) (layer "B.Cu") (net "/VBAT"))
 (segment (start 158.75 93.749999) (end 159.8 94.8) (width 0.6) (layer "B.Cu") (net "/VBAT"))
 (segment (start 159.8 94.8) (end 159.8 101.4) (width 0.6) (layer "B.Cu") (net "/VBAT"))
 (segment (start 156.2 91.2) (end 158.75 93.749999) (width 0.6) (layer "B.Cu") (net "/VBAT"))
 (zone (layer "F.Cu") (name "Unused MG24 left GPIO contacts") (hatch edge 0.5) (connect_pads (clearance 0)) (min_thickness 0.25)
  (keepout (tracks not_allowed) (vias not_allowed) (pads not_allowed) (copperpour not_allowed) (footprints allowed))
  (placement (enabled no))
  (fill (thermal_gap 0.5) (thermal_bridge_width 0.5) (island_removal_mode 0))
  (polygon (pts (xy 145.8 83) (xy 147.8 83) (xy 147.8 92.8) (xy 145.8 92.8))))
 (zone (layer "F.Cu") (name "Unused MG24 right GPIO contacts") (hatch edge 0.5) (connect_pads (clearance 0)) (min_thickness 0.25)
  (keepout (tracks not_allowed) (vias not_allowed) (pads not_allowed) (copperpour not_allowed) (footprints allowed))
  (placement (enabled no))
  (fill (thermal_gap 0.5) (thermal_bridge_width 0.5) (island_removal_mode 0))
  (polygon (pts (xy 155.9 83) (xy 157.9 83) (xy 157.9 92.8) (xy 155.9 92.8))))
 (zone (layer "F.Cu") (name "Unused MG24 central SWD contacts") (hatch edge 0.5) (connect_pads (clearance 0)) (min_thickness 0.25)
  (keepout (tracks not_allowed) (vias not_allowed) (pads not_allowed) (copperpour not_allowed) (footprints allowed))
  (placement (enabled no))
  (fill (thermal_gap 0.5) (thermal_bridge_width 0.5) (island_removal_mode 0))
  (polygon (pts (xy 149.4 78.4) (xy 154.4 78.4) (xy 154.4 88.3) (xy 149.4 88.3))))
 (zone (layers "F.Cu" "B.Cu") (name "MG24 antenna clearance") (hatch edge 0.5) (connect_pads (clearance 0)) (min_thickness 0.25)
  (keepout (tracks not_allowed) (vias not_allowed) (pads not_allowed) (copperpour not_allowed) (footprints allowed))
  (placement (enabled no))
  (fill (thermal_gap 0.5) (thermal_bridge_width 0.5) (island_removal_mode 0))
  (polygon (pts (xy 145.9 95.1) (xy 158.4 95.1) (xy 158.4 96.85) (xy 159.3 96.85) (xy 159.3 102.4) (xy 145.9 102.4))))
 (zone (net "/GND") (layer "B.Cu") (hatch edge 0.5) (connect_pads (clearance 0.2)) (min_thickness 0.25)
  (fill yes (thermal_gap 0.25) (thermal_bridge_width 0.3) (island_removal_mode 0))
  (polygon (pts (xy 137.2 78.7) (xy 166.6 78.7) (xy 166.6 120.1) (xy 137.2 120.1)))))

